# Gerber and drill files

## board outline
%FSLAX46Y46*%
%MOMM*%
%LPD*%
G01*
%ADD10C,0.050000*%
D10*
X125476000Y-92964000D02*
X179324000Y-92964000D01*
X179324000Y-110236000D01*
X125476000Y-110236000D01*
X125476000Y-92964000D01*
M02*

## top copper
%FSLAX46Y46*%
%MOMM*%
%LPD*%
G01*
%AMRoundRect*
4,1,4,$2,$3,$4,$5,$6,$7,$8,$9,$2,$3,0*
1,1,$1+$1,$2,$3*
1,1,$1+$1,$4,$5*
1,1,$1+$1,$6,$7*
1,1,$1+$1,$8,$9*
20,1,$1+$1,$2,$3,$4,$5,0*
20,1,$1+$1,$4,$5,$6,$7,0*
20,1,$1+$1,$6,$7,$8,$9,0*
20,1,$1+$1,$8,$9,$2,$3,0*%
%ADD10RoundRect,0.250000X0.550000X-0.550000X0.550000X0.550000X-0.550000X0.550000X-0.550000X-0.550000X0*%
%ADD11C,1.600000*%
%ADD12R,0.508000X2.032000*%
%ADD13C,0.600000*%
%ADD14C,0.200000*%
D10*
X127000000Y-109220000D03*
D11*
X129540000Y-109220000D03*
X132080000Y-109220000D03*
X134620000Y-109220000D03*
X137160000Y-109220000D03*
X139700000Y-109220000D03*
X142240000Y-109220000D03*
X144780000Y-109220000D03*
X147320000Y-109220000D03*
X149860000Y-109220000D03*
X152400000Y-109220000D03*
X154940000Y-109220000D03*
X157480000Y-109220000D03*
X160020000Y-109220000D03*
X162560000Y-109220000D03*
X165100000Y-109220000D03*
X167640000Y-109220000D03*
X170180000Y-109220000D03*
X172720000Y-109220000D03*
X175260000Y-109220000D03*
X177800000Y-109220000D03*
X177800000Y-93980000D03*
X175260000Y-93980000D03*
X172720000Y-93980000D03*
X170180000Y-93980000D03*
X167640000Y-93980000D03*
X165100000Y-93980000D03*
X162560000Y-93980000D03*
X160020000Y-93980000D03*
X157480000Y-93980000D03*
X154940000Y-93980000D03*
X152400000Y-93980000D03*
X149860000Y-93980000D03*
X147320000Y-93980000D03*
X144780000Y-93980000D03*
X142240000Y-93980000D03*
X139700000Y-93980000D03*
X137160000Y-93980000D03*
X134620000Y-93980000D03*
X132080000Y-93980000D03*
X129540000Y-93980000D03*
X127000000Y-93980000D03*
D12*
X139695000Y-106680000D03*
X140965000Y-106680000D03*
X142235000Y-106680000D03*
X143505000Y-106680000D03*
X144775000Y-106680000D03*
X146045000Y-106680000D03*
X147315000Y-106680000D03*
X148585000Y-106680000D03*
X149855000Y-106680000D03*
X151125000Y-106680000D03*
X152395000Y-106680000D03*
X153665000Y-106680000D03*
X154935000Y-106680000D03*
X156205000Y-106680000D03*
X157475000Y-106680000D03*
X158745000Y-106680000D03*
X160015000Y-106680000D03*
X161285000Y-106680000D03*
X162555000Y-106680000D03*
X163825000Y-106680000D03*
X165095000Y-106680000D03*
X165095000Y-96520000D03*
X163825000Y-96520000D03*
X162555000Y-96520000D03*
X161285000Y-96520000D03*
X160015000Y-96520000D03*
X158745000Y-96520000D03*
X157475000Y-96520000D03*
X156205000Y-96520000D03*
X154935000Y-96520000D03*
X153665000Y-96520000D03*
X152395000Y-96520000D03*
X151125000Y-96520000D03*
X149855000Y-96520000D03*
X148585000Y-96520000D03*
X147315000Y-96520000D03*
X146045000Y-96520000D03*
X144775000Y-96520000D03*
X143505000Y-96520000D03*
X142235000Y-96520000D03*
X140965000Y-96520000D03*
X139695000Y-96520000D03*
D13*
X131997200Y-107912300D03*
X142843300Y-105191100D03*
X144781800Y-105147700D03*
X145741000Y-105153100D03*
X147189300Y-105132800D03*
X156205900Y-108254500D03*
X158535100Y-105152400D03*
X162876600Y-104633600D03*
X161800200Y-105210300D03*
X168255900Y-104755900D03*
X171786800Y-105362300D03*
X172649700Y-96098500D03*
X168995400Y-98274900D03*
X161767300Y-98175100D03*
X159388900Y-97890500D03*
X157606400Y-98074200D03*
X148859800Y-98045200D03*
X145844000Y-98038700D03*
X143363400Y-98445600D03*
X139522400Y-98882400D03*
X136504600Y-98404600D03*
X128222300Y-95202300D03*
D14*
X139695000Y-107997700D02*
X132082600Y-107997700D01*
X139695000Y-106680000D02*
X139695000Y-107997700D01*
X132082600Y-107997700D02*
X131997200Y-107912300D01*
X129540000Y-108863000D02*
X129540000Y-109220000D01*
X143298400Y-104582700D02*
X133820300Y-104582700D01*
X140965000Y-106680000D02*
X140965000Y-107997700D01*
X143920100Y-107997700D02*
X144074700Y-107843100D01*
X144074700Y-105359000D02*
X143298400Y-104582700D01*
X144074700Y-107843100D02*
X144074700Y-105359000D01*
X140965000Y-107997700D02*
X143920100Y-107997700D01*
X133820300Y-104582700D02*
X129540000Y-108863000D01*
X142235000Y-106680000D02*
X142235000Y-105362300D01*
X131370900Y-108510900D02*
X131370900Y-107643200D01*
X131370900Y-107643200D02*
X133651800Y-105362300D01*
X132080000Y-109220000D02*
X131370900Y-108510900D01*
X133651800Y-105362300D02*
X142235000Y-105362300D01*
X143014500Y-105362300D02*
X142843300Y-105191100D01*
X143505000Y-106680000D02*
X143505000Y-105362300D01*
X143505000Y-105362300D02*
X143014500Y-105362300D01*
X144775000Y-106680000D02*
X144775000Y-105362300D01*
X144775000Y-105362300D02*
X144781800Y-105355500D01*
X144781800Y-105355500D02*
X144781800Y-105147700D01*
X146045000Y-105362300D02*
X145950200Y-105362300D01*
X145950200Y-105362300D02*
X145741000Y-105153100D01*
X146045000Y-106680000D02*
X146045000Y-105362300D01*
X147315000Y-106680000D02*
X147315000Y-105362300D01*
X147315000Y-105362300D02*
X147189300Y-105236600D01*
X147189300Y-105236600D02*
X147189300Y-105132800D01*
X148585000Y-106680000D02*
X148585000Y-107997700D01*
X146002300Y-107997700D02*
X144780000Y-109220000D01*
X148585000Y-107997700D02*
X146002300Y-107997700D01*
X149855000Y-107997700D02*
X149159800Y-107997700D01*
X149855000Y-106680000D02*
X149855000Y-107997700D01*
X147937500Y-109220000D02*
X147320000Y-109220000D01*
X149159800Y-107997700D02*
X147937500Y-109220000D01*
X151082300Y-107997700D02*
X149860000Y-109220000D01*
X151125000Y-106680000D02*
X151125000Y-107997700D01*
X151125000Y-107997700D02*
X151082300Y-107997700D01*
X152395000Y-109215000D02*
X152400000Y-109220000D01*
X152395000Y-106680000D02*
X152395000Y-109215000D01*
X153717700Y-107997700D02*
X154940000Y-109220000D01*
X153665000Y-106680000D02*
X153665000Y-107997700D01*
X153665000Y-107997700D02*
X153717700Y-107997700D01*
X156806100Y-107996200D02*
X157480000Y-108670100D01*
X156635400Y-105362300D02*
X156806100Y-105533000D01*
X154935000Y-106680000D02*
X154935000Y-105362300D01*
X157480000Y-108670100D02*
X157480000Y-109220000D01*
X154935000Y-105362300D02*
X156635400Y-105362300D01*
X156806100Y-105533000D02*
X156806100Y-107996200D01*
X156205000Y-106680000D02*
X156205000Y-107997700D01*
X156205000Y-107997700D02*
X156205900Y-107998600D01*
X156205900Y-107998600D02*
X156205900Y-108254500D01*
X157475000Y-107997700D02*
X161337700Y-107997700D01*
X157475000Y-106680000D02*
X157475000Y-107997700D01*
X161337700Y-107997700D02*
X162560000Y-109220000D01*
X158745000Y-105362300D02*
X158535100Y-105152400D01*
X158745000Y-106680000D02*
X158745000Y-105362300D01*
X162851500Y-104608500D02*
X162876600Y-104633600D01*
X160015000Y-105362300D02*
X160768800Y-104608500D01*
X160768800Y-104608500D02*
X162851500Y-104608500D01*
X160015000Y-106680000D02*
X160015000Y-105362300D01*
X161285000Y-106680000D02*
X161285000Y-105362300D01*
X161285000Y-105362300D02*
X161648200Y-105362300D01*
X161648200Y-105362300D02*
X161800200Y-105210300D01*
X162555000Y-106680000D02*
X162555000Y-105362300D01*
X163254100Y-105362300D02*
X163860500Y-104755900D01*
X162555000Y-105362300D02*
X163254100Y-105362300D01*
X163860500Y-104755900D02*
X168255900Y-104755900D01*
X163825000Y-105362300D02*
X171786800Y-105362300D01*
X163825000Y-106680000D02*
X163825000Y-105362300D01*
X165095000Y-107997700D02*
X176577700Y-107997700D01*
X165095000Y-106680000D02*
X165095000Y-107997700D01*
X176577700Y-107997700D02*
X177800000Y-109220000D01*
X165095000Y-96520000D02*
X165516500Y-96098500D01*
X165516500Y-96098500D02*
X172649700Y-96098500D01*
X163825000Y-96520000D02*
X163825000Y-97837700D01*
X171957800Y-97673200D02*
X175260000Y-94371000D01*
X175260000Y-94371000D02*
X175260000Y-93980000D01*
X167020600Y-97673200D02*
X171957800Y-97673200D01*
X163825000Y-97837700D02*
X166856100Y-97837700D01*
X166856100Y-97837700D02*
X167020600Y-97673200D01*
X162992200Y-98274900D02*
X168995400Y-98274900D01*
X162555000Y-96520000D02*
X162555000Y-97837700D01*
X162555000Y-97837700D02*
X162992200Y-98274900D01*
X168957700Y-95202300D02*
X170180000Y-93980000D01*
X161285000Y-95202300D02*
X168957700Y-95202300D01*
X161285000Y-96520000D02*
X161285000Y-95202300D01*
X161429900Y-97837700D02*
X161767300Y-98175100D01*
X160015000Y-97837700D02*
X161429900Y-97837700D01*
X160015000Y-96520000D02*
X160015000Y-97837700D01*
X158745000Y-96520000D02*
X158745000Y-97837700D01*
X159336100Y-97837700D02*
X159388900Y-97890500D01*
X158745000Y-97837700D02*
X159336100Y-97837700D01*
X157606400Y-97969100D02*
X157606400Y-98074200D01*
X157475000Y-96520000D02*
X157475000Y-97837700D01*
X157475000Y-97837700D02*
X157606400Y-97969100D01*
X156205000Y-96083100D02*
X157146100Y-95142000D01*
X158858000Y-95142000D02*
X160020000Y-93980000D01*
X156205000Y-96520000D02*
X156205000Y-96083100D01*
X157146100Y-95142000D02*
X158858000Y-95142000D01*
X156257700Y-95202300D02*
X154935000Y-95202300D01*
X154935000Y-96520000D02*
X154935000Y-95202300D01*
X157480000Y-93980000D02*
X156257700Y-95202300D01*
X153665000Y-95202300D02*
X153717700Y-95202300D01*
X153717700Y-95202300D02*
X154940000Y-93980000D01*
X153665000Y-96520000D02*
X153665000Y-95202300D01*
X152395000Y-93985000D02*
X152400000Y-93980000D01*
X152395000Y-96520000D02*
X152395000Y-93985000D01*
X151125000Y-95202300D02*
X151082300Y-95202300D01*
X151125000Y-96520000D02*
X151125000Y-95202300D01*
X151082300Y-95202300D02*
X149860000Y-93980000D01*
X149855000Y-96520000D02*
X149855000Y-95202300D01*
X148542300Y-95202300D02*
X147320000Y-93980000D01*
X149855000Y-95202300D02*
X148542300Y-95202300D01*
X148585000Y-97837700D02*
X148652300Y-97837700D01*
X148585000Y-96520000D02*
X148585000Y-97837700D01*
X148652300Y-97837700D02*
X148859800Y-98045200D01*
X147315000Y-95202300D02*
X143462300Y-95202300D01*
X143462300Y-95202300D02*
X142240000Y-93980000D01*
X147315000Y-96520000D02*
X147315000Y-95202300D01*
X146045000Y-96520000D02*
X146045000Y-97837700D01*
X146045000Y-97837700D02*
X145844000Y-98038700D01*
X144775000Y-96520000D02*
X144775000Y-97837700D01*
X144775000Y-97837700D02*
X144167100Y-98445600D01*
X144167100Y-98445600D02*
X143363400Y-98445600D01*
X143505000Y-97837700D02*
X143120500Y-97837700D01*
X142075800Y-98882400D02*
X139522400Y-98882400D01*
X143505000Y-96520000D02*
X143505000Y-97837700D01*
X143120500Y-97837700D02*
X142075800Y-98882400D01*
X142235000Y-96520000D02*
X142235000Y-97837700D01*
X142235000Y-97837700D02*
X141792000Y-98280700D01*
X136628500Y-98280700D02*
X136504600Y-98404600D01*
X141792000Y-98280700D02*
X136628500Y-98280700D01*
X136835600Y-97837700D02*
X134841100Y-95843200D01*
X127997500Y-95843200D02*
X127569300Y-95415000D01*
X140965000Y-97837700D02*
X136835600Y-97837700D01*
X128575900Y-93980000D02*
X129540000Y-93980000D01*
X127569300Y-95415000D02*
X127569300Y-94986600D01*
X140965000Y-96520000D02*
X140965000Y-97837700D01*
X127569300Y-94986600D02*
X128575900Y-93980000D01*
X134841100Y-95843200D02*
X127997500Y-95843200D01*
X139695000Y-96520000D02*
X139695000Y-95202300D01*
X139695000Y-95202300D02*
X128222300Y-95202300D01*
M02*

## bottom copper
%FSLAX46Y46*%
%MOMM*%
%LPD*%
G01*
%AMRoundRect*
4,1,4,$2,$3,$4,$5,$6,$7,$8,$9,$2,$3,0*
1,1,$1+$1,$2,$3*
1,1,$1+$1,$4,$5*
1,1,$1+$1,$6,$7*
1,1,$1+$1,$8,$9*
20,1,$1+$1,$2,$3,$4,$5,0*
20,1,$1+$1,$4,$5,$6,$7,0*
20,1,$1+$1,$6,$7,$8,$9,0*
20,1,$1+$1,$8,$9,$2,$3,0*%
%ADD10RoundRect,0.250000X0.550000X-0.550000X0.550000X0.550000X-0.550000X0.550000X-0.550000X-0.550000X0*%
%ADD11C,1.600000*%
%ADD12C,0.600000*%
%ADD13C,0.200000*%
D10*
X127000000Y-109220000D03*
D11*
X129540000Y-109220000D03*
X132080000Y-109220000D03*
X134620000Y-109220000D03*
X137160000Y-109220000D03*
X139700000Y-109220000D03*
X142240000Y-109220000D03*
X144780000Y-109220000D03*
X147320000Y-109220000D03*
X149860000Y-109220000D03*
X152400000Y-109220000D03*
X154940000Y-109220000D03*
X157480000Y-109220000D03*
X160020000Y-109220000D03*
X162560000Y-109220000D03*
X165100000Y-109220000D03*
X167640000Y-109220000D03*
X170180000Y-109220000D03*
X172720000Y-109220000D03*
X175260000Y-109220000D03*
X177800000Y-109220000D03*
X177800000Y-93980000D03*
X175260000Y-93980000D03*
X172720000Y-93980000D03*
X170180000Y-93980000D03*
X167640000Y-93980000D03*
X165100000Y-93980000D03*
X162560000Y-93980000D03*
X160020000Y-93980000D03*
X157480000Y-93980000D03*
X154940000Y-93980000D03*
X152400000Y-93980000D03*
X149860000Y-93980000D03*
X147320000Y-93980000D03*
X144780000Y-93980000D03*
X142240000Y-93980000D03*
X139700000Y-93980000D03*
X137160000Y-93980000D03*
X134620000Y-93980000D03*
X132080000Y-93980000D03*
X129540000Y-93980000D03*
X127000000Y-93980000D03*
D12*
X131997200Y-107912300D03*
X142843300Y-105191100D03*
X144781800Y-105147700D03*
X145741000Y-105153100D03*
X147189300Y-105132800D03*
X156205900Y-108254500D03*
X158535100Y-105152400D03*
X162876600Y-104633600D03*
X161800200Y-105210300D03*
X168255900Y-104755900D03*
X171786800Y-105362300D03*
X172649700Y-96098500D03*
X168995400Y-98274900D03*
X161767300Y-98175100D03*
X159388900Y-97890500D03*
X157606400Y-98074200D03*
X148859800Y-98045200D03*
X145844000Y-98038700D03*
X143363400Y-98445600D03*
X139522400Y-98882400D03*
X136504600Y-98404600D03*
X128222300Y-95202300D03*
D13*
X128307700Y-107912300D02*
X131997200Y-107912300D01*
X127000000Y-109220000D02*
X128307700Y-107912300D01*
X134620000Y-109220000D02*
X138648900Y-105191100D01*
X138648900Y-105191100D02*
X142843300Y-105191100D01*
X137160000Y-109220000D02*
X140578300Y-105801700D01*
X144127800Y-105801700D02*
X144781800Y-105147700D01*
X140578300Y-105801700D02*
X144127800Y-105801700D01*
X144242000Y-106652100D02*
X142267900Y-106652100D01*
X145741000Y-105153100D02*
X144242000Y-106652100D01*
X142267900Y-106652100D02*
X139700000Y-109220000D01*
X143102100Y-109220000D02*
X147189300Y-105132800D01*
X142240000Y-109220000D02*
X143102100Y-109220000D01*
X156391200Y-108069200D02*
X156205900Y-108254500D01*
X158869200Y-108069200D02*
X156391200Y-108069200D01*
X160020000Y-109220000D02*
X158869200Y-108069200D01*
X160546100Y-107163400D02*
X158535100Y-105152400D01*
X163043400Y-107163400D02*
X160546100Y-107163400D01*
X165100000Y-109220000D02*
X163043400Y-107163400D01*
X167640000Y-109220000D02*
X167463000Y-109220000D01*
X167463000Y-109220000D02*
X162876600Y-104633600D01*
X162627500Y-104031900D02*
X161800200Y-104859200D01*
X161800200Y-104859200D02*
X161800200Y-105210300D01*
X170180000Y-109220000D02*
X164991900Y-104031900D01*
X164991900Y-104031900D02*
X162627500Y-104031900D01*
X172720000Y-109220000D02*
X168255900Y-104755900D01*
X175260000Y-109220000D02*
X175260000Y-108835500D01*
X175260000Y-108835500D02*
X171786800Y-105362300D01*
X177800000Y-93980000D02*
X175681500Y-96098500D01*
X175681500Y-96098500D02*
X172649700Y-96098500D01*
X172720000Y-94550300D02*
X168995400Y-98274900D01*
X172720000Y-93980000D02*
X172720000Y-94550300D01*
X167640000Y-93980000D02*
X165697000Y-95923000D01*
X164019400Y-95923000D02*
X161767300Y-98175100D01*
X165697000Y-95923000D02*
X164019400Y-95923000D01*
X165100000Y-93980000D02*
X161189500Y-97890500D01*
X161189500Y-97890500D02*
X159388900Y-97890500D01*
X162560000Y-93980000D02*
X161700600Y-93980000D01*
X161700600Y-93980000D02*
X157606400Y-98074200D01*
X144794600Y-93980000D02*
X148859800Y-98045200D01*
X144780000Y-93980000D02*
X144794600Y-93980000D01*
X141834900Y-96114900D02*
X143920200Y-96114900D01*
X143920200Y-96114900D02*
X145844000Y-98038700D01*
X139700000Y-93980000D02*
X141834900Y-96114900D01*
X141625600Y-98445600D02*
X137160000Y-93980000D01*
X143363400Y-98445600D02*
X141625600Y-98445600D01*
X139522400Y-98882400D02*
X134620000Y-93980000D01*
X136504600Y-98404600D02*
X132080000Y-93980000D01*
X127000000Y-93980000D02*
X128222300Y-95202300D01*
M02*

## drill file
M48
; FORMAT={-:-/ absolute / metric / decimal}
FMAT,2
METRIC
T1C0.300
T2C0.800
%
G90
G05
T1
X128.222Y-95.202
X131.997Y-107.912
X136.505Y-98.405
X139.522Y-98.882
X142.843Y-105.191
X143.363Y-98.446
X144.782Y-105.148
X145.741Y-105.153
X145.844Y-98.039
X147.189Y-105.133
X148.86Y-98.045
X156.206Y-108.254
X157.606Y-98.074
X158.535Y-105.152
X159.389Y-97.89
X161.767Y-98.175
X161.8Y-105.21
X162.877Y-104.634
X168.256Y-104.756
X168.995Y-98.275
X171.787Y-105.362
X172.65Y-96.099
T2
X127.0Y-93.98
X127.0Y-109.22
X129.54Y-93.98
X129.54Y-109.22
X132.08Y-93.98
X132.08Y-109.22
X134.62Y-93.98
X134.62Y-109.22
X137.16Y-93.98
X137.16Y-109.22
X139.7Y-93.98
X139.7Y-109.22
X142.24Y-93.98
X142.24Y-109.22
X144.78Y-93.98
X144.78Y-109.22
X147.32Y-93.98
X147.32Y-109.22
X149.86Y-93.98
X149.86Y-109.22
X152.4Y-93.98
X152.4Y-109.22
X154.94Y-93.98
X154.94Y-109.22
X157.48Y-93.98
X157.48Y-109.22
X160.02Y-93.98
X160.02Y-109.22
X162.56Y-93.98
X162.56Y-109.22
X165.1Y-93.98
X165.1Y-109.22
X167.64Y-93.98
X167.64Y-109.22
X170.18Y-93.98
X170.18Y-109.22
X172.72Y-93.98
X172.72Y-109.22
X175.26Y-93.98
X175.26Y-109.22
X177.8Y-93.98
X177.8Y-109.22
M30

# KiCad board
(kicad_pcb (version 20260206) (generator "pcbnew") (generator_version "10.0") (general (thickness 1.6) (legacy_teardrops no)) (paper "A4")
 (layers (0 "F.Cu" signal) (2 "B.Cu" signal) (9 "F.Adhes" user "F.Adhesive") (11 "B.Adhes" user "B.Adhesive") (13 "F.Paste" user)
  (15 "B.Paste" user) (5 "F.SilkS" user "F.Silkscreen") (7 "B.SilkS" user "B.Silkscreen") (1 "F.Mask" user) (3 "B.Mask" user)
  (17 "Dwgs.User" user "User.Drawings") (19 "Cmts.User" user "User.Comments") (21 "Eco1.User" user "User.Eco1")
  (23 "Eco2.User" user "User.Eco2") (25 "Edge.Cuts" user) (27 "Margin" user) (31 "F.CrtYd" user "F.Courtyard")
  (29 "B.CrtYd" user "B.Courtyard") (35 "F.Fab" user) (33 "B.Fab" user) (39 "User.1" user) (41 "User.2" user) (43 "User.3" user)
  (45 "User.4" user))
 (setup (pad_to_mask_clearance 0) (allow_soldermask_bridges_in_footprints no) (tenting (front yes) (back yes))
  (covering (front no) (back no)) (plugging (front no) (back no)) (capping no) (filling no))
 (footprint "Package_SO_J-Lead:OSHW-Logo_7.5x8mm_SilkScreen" (layer "F.Cu") (at 152.5 101.5)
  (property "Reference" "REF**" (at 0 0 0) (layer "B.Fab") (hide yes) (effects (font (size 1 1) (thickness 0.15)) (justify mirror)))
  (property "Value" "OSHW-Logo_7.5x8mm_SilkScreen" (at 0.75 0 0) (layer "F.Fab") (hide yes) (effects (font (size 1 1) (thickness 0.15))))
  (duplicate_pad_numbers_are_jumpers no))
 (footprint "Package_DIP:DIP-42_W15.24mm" (layer "F.Cu") (at 127 109.22 90)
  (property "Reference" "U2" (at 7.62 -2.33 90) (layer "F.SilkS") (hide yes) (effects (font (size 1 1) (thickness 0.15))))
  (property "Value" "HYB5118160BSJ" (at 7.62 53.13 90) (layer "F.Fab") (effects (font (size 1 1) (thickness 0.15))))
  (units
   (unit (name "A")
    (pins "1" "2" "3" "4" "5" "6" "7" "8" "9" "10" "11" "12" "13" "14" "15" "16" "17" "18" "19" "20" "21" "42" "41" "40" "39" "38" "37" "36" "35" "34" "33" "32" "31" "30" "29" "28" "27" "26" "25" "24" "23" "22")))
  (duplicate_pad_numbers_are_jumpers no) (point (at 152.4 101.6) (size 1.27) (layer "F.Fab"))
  (pad "1" thru_hole roundrect (at 0 0 90) (size 1.6 1.6) (drill 0.8) (layers "*.Cu" "*.Mask") (remove_unused_layers no)
   (roundrect_rratio 0.15625) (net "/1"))
  (pad "2" thru_hole circle (at 0 2.54 90) (size 1.6 1.6) (drill 0.8) (layers "*.Cu" "*.Mask") (remove_unused_layers no) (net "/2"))
  (pad "3" thru_hole circle (at 0 5.08 90) (size 1.6 1.6) (drill 0.8) (layers "*.Cu" "*.Mask") (remove_unused_layers no) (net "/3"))
  (pad "4" thru_hole circle (at 0 7.62 90) (size 1.6 1.6) (drill 0.8) (layers "*.Cu" "*.Mask") (remove_unused_layers no) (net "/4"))
  (pad "5" thru_hole circle (at 0 10.16 90) (size 1.6 1.6) (drill 0.8) (layers "*.Cu" "*.Mask") (remove_unused_layers no) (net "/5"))
  (pad "6" thru_hole circle (at 0 12.7 90) (size 1.6 1.6) (drill 0.8) (layers "*.Cu" "*.Mask") (remove_unused_layers no) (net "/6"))
  (pad "7" thru_hole circle (at 0 15.24 90) (size 1.6 1.6) (drill 0.8) (layers "*.Cu" "*.Mask") (remove_unused_layers no) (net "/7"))
  (pad "8" thru_hole circle (at 0 17.78 90) (size 1.6 1.6) (drill 0.8) (layers "*.Cu" "*.Mask") (remove_unused_layers no) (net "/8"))
  (pad "9" thru_hole circle (at 0 20.32 90) (size 1.6 1.6) (drill 0.8) (layers "*.Cu" "*.Mask") (remove_unused_layers no) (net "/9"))
  (pad "10" thru_hole circle (at 0 22.86 90) (size 1.6 1.6) (drill 0.8) (layers "*.Cu" "*.Mask") (remove_unused_layers no) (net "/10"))
  (pad "11" thru_hole circle (at 0 25.4 90) (size 1.6 1.6) (drill 0.8) (layers "*.Cu" "*.Mask") (remove_unused_layers no) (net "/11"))
  (pad "12" thru_hole circle (at 0 27.94 90) (size 1.6 1.6) (drill 0.8) (layers "*.Cu" "*.Mask") (remove_unused_layers no) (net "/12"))
  (pad "13" thru_hole circle (at 0 30.48 90) (size 1.6 1.6) (drill 0.8) (layers "*.Cu" "*.Mask") (remove_unused_layers no) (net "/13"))
  (pad "14" thru_hole circle (at 0 33.02 90) (size 1.6 1.6) (drill 0.8) (layers "*.Cu" "*.Mask") (remove_unused_layers no) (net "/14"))
  (pad "15" thru_hole circle (at 0 35.56 90) (size 1.6 1.6) (drill 0.8) (layers "*.Cu" "*.Mask") (remove_unused_layers no) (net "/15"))
  (pad "16" thru_hole circle (at 0 38.1 90) (size 1.6 1.6) (drill 0.8) (layers "*.Cu" "*.Mask") (remove_unused_layers no) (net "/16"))
  (pad "17" thru_hole circle (at 0 40.64 90) (size 1.6 1.6) (drill 0.8) (layers "*.Cu" "*.Mask") (remove_unused_layers no) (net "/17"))
  (pad "18" thru_hole circle (at 0 43.18 90) (size 1.6 1.6) (drill 0.8) (layers "*.Cu" "*.Mask") (remove_unused_layers no) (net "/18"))
  (pad "19" thru_hole circle (at 0 45.72 90) (size 1.6 1.6) (drill 0.8) (layers "*.Cu" "*.Mask") (remove_unused_layers no) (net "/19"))
  (pad "20" thru_hole circle (at 0 48.26 90) (size 1.6 1.6) (drill 0.8) (layers "*.Cu" "*.Mask") (remove_unused_layers no) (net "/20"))
  (pad "21" thru_hole circle (at 0 50.8 90) (size 1.6 1.6) (drill 0.8) (layers "*.Cu" "*.Mask") (remove_unused_layers no) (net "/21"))
  (pad "22" thru_hole circle (at 15.24 50.8 90) (size 1.6 1.6) (drill 0.8) (layers "*.Cu" "*.Mask") (remove_unused_layers no) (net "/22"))
  (pad "23" thru_hole circle (at 15.24 48.26 90) (size 1.6 1.6) (drill 0.8) (layers "*.Cu" "*.Mask") (remove_unused_layers no) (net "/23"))
  (pad "24" thru_hole circle (at 15.24 45.72 90) (size 1.6 1.6) (drill 0.8) (layers "*.Cu" "*.Mask") (remove_unused_layers no) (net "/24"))
  (pad "25" thru_hole circle (at 15.24 43.18 90) (size 1.6 1.6) (drill 0.8) (layers "*.Cu" "*.Mask") (remove_unused_layers no) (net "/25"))
  (pad "26" thru_hole circle (at 15.24 40.64 90) (size 1.6 1.6) (drill 0.8) (layers "*.Cu" "*.Mask") (remove_unused_layers no) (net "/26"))
  (pad "27" thru_hole circle (at 15.24 38.1 90) (size 1.6 1.6) (drill 0.8) (layers "*.Cu" "*.Mask") (remove_unused_layers no) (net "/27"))
  (pad "28" thru_hole circle (at 15.24 35.56 90) (size 1.6 1.6) (drill 0.8) (layers "*.Cu" "*.Mask") (remove_unused_layers no) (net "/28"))
  (pad "29" thru_hole circle (at 15.24 33.02 90) (size 1.6 1.6) (drill 0.8) (layers "*.Cu" "*.Mask") (remove_unused_layers no) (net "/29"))
  (pad "30" thru_hole circle (at 15.24 30.48 90) (size 1.6 1.6) (drill 0.8) (layers "*.Cu" "*.Mask") (remove_unused_layers no) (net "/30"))
  (pad "31" thru_hole circle (at 15.24 27.94 90) (size 1.6 1.6) (drill 0.8) (layers "*.Cu" "*.Mask") (remove_unused_layers no) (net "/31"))
  (pad "32" thru_hole circle (at 15.24 25.4 90) (size 1.6 1.6) (drill 0.8) (layers "*.Cu" "*.Mask") (remove_unused_layers no) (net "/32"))
  (pad "33" thru_hole circle (at 15.24 22.86 90) (size 1.6 1.6) (drill 0.8) (layers "*.Cu" "*.Mask") (remove_unused_layers no) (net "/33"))
  (pad "34" thru_hole circle (at 15.24 20.32 90) (size 1.6 1.6) (drill 0.8) (layers "*.Cu" "*.Mask") (remove_unused_layers no) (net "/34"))
  (pad "35" thru_hole circle (at 15.24 17.78 90) (size 1.6 1.6) (drill 0.8) (layers "*.Cu" "*.Mask") (remove_unused_layers no) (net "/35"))
  (pad "36" thru_hole circle (at 15.24 15.24 90) (size 1.6 1.6) (drill 0.8) (layers "*.Cu" "*.Mask") (remove_unused_layers no) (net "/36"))
  (pad "37" thru_hole circle (at 15.24 12.7 90) (size 1.6 1.6) (drill 0.8) (layers "*.Cu" "*.Mask") (remove_unused_layers no) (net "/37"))
  (pad "38" thru_hole circle (at 15.24 10.16 90) (size 1.6 1.6) (drill 0.8) (layers "*.Cu" "*.Mask") (remove_unused_layers no) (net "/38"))
  (pad "39" thru_hole circle (at 15.24 7.62 90) (size 1.6 1.6) (drill 0.8) (layers "*.Cu" "*.Mask") (remove_unused_layers no) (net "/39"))
  (pad "40" thru_hole circle (at 15.24 5.08 90) (size 1.6 1.6) (drill 0.8) (layers "*.Cu" "*.Mask") (remove_unused_layers no) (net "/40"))
  (pad "41" thru_hole circle (at 15.24 2.54 90) (size 1.6 1.6) (drill 0.8) (layers "*.Cu" "*.Mask") (remove_unused_layers no) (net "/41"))
  (pad "42" thru_hole circle (at 15.24 0 90) (size 1.6 1.6) (drill 0.8) (layers "*.Cu" "*.Mask") (remove_unused_layers no) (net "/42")))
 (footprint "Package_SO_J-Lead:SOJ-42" (layer "F.Cu") (at 152.395 101.6)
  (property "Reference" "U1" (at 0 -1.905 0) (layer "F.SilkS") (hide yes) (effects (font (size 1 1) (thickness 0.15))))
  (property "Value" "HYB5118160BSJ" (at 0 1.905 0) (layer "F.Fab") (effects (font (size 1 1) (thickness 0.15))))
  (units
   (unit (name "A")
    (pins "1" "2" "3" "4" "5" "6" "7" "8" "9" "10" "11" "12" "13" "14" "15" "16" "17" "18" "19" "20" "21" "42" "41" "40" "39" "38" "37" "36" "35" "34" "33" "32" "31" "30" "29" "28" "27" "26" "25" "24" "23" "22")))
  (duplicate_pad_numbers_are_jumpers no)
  (pad "1" smd rect (at -12.7 5.08) (size 0.508 2.032) (layers "F.Cu" "F.Mask" "F.Paste") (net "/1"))
  (pad "2" smd rect (at -11.43 5.08) (size 0.508 2.032) (layers "F.Cu" "F.Mask" "F.Paste") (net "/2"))
  (pad "3" smd rect (at -10.16 5.08) (size 0.508 2.032) (layers "F.Cu" "F.Mask" "F.Paste") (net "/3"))
  (pad "4" smd rect (at -8.89 5.08) (size 0.508 2.032) (layers "F.Cu" "F.Mask" "F.Paste") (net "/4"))
  (pad "5" smd rect (at -7.62 5.08) (size 0.508 2.032) (layers "F.Cu" "F.Mask" "F.Paste") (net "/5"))
  (pad "6" smd rect (at -6.35 5.08) (size 0.508 2.032) (layers "F.Cu" "F.Mask" "F.Paste") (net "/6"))
  (pad "7" smd rect (at -5.08 5.08) (size 0.508 2.032) (layers "F.Cu" "F.Mask" "F.Paste") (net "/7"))
  (pad "8" smd rect (at -3.81 5.08) (size 0.508 2.032) (layers "F.Cu" "F.Mask" "F.Paste") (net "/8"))
  (pad "9" smd rect (at -2.54 5.08) (size 0.508 2.032) (layers "F.Cu" "F.Mask" "F.Paste") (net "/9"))
  (pad "10" smd rect (at -1.27 5.08) (size 0.508 2.032) (layers "F.Cu" "F.Mask" "F.Paste") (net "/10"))
  (pad "11" smd rect (at 0 5.08) (size 0.508 2.032) (layers "F.Cu" "F.Mask" "F.Paste") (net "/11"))
  (pad "12" smd rect (at 1.27 5.08) (size 0.508 2.032) (layers "F.Cu" "F.Mask" "F.Paste") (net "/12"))
  (pad "13" smd rect (at 2.54 5.08) (size 0.508 2.032) (layers "F.Cu" "F.Mask" "F.Paste") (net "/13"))
  (pad "14" smd rect (at 3.81 5.08) (size 0.508 2.032) (layers "F.Cu" "F.Mask" "F.Paste") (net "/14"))
  (pad "15" smd rect (at 5.08 5.08) (size 0.508 2.032) (layers "F.Cu" "F.Mask" "F.Paste") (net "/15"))
  (pad "16" smd rect (at 6.35 5.08) (size 0.508 2.032) (layers "F.Cu" "F.Mask" "F.Paste") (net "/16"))
  (pad "17" smd rect (at 7.62 5.08) (size 0.508 2.032) (layers "F.Cu" "F.Mask" "F.Paste") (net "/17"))
  (pad "18" smd rect (at 8.89 5.08) (size 0.508 2.032) (layers "F.Cu" "F.Mask" "F.Paste") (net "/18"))
  (pad "19" smd rect (at 10.16 5.08) (size 0.508 2.032) (layers "F.Cu" "F.Mask" "F.Paste") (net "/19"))
  (pad "20" smd rect (at 11.43 5.08) (size 0.508 2.032) (layers "F.Cu" "F.Mask" "F.Paste") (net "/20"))
  (pad "21" smd rect (at 12.7 5.08) (size 0.508 2.032) (layers "F.Cu" "F.Mask" "F.Paste") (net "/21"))
  (pad "22" smd rect (at 12.7 -5.08) (size 0.508 2.032) (layers "F.Cu" "F.Mask" "F.Paste") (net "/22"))
  (pad "23" smd rect (at 11.43 -5.08) (size 0.508 2.032) (layers "F.Cu" "F.Mask" "F.Paste") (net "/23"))
  (pad "24" smd rect (at 10.16 -5.08) (size 0.508 2.032) (layers "F.Cu" "F.Mask" "F.Paste") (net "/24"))
  (pad "25" smd rect (at 8.89 -5.08) (size 0.508 2.032) (layers "F.Cu" "F.Mask" "F.Paste") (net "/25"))
  (pad "26" smd rect (at 7.62 -5.08) (size 0.508 2.032) (layers "F.Cu" "F.Mask" "F.Paste") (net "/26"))
  (pad "27" smd rect (at 6.35 -5.08) (size 0.508 2.032) (layers "F.Cu" "F.Mask" "F.Paste") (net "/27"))
  (pad "28" smd rect (at 5.08 -5.08) (size 0.508 2.032) (layers "F.Cu" "F.Mask" "F.Paste") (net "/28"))
  (pad "29" smd rect (at 3.81 -5.08) (size 0.508 2.032) (layers "F.Cu" "F.Mask" "F.Paste") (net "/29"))
  (pad "30" smd rect (at 2.54 -5.08) (size 0.508 2.032) (layers "F.Cu" "F.Mask" "F.Paste") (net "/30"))
  (pad "31" smd rect (at 1.27 -5.08) (size 0.508 2.032) (layers "F.Cu" "F.Mask" "F.Paste") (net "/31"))
  (pad "32" smd rect (at 0 -5.08) (size 0.508 2.032) (layers "F.Cu" "F.Mask" "F.Paste") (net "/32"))
  (pad "33" smd rect (at -1.27 -5.08) (size 0.508 2.032) (layers "F.Cu" "F.Mask" "F.Paste") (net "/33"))
  (pad "34" smd rect (at -2.54 -5.08) (size 0.508 2.032) (layers "F.Cu" "F.Mask" "F.Paste") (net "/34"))
  (pad "35" smd rect (at -3.81 -5.08) (size 0.508 2.032) (layers "F.Cu" "F.Mask" "F.Paste") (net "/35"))
  (pad "36" smd rect (at -5.08 -5.08) (size 0.508 2.032) (layers "F.Cu" "F.Mask" "F.Paste") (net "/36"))
  (pad "37" smd rect (at -6.35 -5.08) (size 0.508 2.032) (layers "F.Cu" "F.Mask" "F.Paste") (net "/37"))
  (pad "38" smd rect (at -7.62 -5.08) (size 0.508 2.032) (layers "F.Cu" "F.Mask" "F.Paste") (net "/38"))
  (pad "39" smd rect (at -8.89 -5.08) (size 0.508 2.032) (layers "F.Cu" "F.Mask" "F.Paste") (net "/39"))
  (pad "40" smd rect (at -10.16 -5.08) (size 0.508 2.032) (layers "F.Cu" "F.Mask" "F.Paste") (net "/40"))
  (pad "41" smd rect (at -11.43 -5.08) (size 0.508 2.032) (layers "F.Cu" "F.Mask" "F.Paste") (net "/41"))
  (pad "42" smd rect (at -12.7 -5.08) (size 0.508 2.032) (layers "F.Cu" "F.Mask" "F.Paste") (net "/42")))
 (gr_rect (start 125.476 92.964) (end 179.324 110.236) (stroke (width 0.05) (type default)) (fill no) (layer "Edge.Cuts"))
 (segment (start 139.695 107.9977) (end 132.0826 107.9977) (width 0.2) (layer "F.Cu") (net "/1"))
 (segment (start 139.695 106.68) (end 139.695 107.9977) (width 0.2) (layer "F.Cu") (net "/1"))
 (segment (start 132.0826 107.9977) (end 131.9972 107.9123) (width 0.2) (layer "F.Cu") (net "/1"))
 (via (at 131.9972 107.9123) (size 0.6) (drill 0.3) (layers "F.Cu" "B.Cu") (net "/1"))
 (segment (start 128.3077 107.9123) (end 131.9972 107.9123) (width 0.2) (layer "B.Cu") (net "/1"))
 (segment (start 127 109.22) (end 128.3077 107.9123) (width 0.2) (layer "B.Cu") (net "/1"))
 (segment (start 129.54 108.863) (end 129.54 109.22) (width 0.2) (layer "F.Cu") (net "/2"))
 (segment (start 143.2984 104.5827) (end 133.8203 104.5827) (width 0.2) (layer "F.Cu") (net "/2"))
 (segment (start 140.965 106.68) (end 140.965 107.9977) (width 0.2) (layer "F.Cu") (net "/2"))
 (segment (start 143.9201 107.9977) (end 144.0747 107.8431) (width 0.2) (layer "F.Cu") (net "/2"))
 (segment (start 144.0747 105.359) (end 143.2984 104.5827) (width 0.2) (layer "F.Cu") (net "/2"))
 (segment (start 144.0747 107.8431) (end 144.0747 105.359) (width 0.2) (layer "F.Cu") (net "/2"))
 (segment (start 140.965 107.9977) (end 143.9201 107.9977) (width 0.2) (layer "F.Cu") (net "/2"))
 (segment (start 133.8203 104.5827) (end 129.54 108.863) (width 0.2) (layer "F.Cu") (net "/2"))
 (segment (start 142.235 106.68) (end 142.235 105.3623) (width 0.2) (layer "F.Cu") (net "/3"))
 (segment (start 131.3709 108.5109) (end 131.3709 107.6432) (width 0.2) (layer "F.Cu") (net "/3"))
 (segment (start 131.3709 107.6432) (end 133.6518 105.3623) (width 0.2) (layer "F.Cu") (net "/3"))
 (segment (start 132.08 109.22) (end 131.3709 108.5109) (width 0.2) (layer "F.Cu") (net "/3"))
 (segment (start 133.6518 105.3623) (end 142.235 105.3623) (width 0.2) (layer "F.Cu") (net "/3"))
 (segment (start 143.0145 105.3623) (end 142.8433 105.1911) (width 0.2) (layer "F.Cu") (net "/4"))
 (segment (start 143.505 106.68) (end 143.505 105.3623) (width 0.2) (layer "F.Cu") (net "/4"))
 (segment (start 143.505 105.3623) (end 143.0145 105.3623) (width 0.2) (layer "F.Cu") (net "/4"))
 (via (at 142.8433 105.1911) (size 0.6) (drill 0.3) (layers "F.Cu" "B.Cu") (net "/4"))
 (segment (start 134.62 109.22) (end 138.6489 105.1911) (width 0.2) (layer "B.Cu") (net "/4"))
 (segment (start 138.6489 105.1911) (end 142.8433 105.1911) (width 0.2) (layer "B.Cu") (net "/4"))
 (segment (start 144.775 106.68) (end 144.775 105.3623) (width 0.2) (layer "F.Cu") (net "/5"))
 (segment (start 144.775 105.3623) (end 144.7818 105.3555) (width 0.2) (layer "F.Cu") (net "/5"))
 (segment (start 144.7818 105.3555) (end 144.7818 105.1477) (width 0.2) (layer "F.Cu") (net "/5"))
 (via (at 144.7818 105.1477) (size 0.6) (drill 0.3) (layers "F.Cu" "B.Cu") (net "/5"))
 (segment (start 137.16 109.22) (end 140.5783 105.8017) (width 0.2) (layer "B.Cu") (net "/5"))
 (segment (start 144.1278 105.8017) (end 144.7818 105.1477) (width 0.2) (layer "B.Cu") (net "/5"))
 (segment (start 140.5783 105.8017) (end 144.1278 105.8017) (width 0.2) (layer "B.Cu") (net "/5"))
 (segment (start 146.045 105.3623) (end 145.9502 105.3623) (width 0.2) (layer "F.Cu") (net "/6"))
 (segment (start 145.9502 105.3623) (end 145.741 105.1531) (width 0.2) (layer "F.Cu") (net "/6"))
 (segment (start 146.045 106.68) (end 146.045 105.3623) (width 0.2) (layer "F.Cu") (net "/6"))
 (via (at 145.741 105.1531) (size 0.6) (drill 0.3) (layers "F.Cu" "B.Cu") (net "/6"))
 (segment (start 144.242 106.6521) (end 142.2679 106.6521) (width 0.2) (layer "B.Cu") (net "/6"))
 (segment (start 145.741 105.1531) (end 144.242 106.6521) (width 0.2) (layer "B.Cu") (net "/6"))
 (segment (start 142.2679 106.6521) (end 139.7 109.22) (width 0.2) (layer "B.Cu") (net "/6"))
 (segment (start 147.315 106.68) (end 147.315 105.3623) (width 0.2) (layer "F.Cu") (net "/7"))
 (segment (start 147.315 105.3623) (end 147.1893 105.2366) (width 0.2) (layer "F.Cu") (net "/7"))
 (segment (start 147.1893 105.2366) (end 147.1893 105.1328) (width 0.2) (layer "F.Cu") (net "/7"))
 (via (at 147.1893 105.1328) (size 0.6) (drill 0.3) (layers "F.Cu" "B.Cu") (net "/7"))
 (segment (start 143.1021 109.22) (end 147.1893 105.1328) (width 0.2) (layer "B.Cu") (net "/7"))
 (segment (start 142.24 109.22) (end 143.1021 109.22) (width 0.2) (layer "B.Cu") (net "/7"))
 (segment (start 148.585 106.68) (end 148.585 107.9977) (width 0.2) (layer "F.Cu") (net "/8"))
 (segment (start 146.0023 107.9977) (end 144.78 109.22) (width 0.2) (layer "F.Cu") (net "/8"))
 (segment (start 148.585 107.9977) (end 146.0023 107.9977) (width 0.2) (layer "F.Cu") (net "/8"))
 (segment (start 149.855 107.9977) (end 149.1598 107.9977) (width 0.2) (layer "F.Cu") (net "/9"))
 (segment (start 149.855 106.68) (end 149.855 107.9977) (width 0.2) (layer "F.Cu") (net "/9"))
 (segment (start 147.9375 109.22) (end 147.32 109.22) (width 0.2) (layer "F.Cu") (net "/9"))
 (segment (start 149.1598 107.9977) (end 147.9375 109.22) (width 0.2) (layer "F.Cu") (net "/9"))
 (segment (start 151.0823 107.9977) (end 149.86 109.22) (width 0.2) (layer "F.Cu") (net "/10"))
 (segment (start 151.125 106.68) (end 151.125 107.9977) (width 0.2) (layer "F.Cu") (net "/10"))
 (segment (start 151.125 107.9977) (end 151.0823 107.9977) (width 0.2) (layer "F.Cu") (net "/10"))
 (segment (start 152.395 109.215) (end 152.4 109.22) (width 0.2) (layer "F.Cu") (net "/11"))
 (segment (start 152.395 106.68) (end 152.395 109.215) (width 0.2) (layer "F.Cu") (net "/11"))
 (segment (start 153.7177 107.9977) (end 154.94 109.22) (width 0.2) (layer "F.Cu") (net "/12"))
 (segment (start 153.665 106.68) (end 153.665 107.9977) (width 0.2) (layer "F.Cu") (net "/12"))
 (segment (start 153.665 107.9977) (end 153.7177 107.9977) (width 0.2) (layer "F.Cu") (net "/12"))
 (segment (start 156.8061 107.9962) (end 157.48 108.6701) (width 0.2) (layer "F.Cu") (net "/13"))
 (segment (start 156.6354 105.3623) (end 156.8061 105.533) (width 0.2) (layer "F.Cu") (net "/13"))
 (segment (start 154.935 106.68) (end 154.935 105.3623) (width 0.2) (layer "F.Cu") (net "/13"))
 (segment (start 157.48 108.6701) (end 157.48 109.22) (width 0.2) (layer "F.Cu") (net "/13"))
 (segment (start 154.935 105.3623) (end 156.6354 105.3623) (width 0.2) (layer "F.Cu") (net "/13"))
 (segment (start 156.8061 105.533) (end 156.8061 107.9962) (width 0.2) (layer "F.Cu") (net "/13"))
 (segment (start 156.205 106.68) (end 156.205 107.9977) (width 0.2) (layer "F.Cu") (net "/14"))
 (segment (start 156.205 107.9977) (end 156.2059 107.9986) (width 0.2) (layer "F.Cu") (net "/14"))
 (segment (start 156.2059 107.9986) (end 156.2059 108.2545) (width 0.2) (layer "F.Cu") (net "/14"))
 (via (at 156.2059 108.2545) (size 0.6) (drill 0.3) (layers "F.Cu" "B.Cu") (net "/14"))
 (segment (start 156.3912 108.0692) (end 156.2059 108.2545) (width 0.2) (layer "B.Cu") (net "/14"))
 (segment (start 158.8692 108.0692) (end 156.3912 108.0692) (width 0.2) (layer "B.Cu") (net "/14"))
 (segment (start 160.02 109.22) (end 158.8692 108.0692) (width 0.2) (layer "B.Cu") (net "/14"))
 (segment (start 157.475 107.9977) (end 161.3377 107.9977) (width 0.2) (layer "F.Cu") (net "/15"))
 (segment (start 157.475 106.68) (end 157.475 107.9977) (width 0.2) (layer "F.Cu") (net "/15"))
 (segment (start 161.3377 107.9977) (end 162.56 109.22) (width 0.2) (layer "F.Cu") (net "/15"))
 (segment (start 158.745 105.3623) (end 158.5351 105.1524) (width 0.2) (layer "F.Cu") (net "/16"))
 (segment (start 158.745 106.68) (end 158.745 105.3623) (width 0.2) (layer "F.Cu") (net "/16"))
 (via (at 158.5351 105.1524) (size 0.6) (drill 0.3) (layers "F.Cu" "B.Cu") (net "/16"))
 (segment (start 160.5461 107.1634) (end 158.5351 105.1524) (width 0.2) (layer "B.Cu") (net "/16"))
 (segment (start 163.0434 107.1634) (end 160.5461 107.1634) (width 0.2) (layer "B.Cu") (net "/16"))
 (segment (start 165.1 109.22) (end 163.0434 107.1634) (width 0.2) (layer "B.Cu") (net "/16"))
 (segment (start 162.8515 104.6085) (end 162.8766 104.6336) (width 0.2) (layer "F.Cu") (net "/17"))
 (segment (start 160.015 105.3623) (end 160.7688 104.6085) (width 0.2) (layer "F.Cu") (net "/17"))
 (segment (start 160.7688 104.6085) (end 162.8515 104.6085) (width 0.2) (layer "F.Cu") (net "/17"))
 (segment (start 160.015 106.68) (end 160.015 105.3623) (width 0.2) (layer "F.Cu") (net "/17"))
 (via (at 162.8766 104.6336) (size 0.6) (drill 0.3) (layers "F.Cu" "B.Cu") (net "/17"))
 (segment (start 167.64 109.22) (end 167.463 109.22) (width 0.2) (layer "B.Cu") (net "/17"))
 (segment (start 167.463 109.22) (end 162.8766 104.6336) (width 0.2) (layer "B.Cu") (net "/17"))
 (segment (start 161.285 106.68) (end 161.285 105.3623) (width 0.2) (layer "F.Cu") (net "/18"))
 (segment (start 161.285 105.3623) (end 161.6482 105.3623) (width 0.2) (layer "F.Cu") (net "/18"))
 (segment (start 161.6482 105.3623) (end 161.8002 105.2103) (width 0.2) (layer "F.Cu") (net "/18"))
 (via (at 161.8002 105.2103) (size 0.6) (drill 0.3) (layers "F.Cu" "B.Cu") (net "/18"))
 (segment (start 162.6275 104.0319) (end 161.8002 104.8592) (width 0.2) (layer "B.Cu") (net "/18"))
 (segment (start 161.8002 104.8592) (end 161.8002 105.2103) (width 0.2) (layer "B.Cu") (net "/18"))
 (segment (start 170.18 109.22) (end 164.9919 104.0319) (width 0.2) (layer "B.Cu") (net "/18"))
 (segment (start 164.9919 104.0319) (end 162.6275 104.0319) (width 0.2) (layer "B.Cu") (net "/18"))
 (segment (start 162.555 106.68) (end 162.555 105.3623) (width 0.2) (layer "F.Cu") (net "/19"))
 (segment (start 163.2541 105.3623) (end 163.8605 104.7559) (width 0.2) (layer "F.Cu") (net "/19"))
 (segment (start 162.555 105.3623) (end 163.2541 105.3623) (width 0.2) (layer "F.Cu") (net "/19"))
 (segment (start 163.8605 104.7559) (end 168.2559 104.7559) (width 0.2) (layer "F.Cu") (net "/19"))
 (via (at 168.2559 104.7559) (size 0.6) (drill 0.3) (layers "F.Cu" "B.Cu") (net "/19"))
 (segment (start 172.72 109.22) (end 168.2559 104.7559) (width 0.2) (layer "B.Cu") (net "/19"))
 (segment (start 163.825 105.3623) (end 171.7868 105.3623) (width 0.2) (layer "F.Cu") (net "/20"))
 (segment (start 163.825 106.68) (end 163.825 105.3623) (width 0.2) (layer "F.Cu") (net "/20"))
 (via (at 171.7868 105.3623) (size 0.6) (drill 0.3) (layers "F.Cu" "B.Cu") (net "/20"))
 (segment (start 175.26 109.22) (end 175.26 108.8355) (width 0.2) (layer "B.Cu") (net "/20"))
 (segment (start 175.26 108.8355) (end 171.7868 105.3623) (width 0.2) (layer "B.Cu") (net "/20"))
 (segment (start 165.095 107.9977) (end 176.5777 107.9977) (width 0.2) (layer "F.Cu") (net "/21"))
 (segment (start 165.095 106.68) (end 165.095 107.9977) (width 0.2) (layer "F.Cu") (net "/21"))
 (segment (start 176.5777 107.9977) (end 177.8 109.22) (width 0.2) (layer "F.Cu") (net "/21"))
 (segment (start 165.095 96.52) (end 165.5165 96.0985) (width 0.2) (layer "F.Cu") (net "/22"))
 (segment (start 165.5165 96.0985) (end 172.6497 96.0985) (width 0.2) (layer "F.Cu") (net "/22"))
 (via (at 172.6497 96.0985) (size 0.6) (drill 0.3) (layers "F.Cu" "B.Cu") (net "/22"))
 (segment (start 177.8 93.98) (end 175.6815 96.0985) (width 0.2) (layer "B.Cu") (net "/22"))
 (segment (start 175.6815 96.0985) (end 172.6497 96.0985) (width 0.2) (layer "B.Cu") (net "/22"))
 (segment (start 163.825 96.52) (end 163.825 97.8377) (width 0.2) (layer "F.Cu") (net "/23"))
 (segment (start 171.9578 97.6732) (end 175.26 94.371) (width 0.2) (layer "F.Cu") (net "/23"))
 (segment (start 175.26 94.371) (end 175.26 93.98) (width 0.2) (layer "F.Cu") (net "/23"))
 (segment (start 167.0206 97.6732) (end 171.9578 97.6732) (width 0.2) (layer "F.Cu") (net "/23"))
 (segment (start 163.825 97.8377) (end 166.8561 97.8377) (width 0.2) (layer "F.Cu") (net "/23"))
 (segment (start 166.8561 97.8377) (end 167.0206 97.6732) (width 0.2) (layer "F.Cu") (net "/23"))
 (segment (start 162.9922 98.2749) (end 168.9954 98.2749) (width 0.2) (layer "F.Cu") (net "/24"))
 (segment (start 162.555 96.52) (end 162.555 97.8377) (width 0.2) (layer "F.Cu") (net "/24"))
 (segment (start 162.555 97.8377) (end 162.9922 98.2749) (width 0.2) (layer "F.Cu") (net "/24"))
 (via (at 168.9954 98.2749) (size 0.6) (drill 0.3) (layers "F.Cu" "B.Cu") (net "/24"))
 (segment (start 172.72 94.5503) (end 168.9954 98.2749) (width 0.2) (layer "B.Cu") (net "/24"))
 (segment (start 172.72 93.98) (end 172.72 94.5503) (width 0.2) (layer "B.Cu") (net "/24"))
 (segment (start 168.9577 95.2023) (end 170.18 93.98) (width 0.2) (layer "F.Cu") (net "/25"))
 (segment (start 161.285 95.2023) (end 168.9577 95.2023) (width 0.2) (layer "F.Cu") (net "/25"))
 (segment (start 161.285 96.52) (end 161.285 95.2023) (width 0.2) (layer "F.Cu") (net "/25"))
 (segment (start 161.4299 97.8377) (end 161.7673 98.1751) (width 0.2) (layer "F.Cu") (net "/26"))
 (segment (start 160.015 97.8377) (end 161.4299 97.8377) (width 0.2) (layer "F.Cu") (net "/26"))
 (segment (start 160.015 96.52) (end 160.015 97.8377) (width 0.2) (layer "F.Cu") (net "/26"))
 (via (at 161.7673 98.1751) (size 0.6) (drill 0.3) (layers "F.Cu" "B.Cu") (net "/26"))
 (segment (start 167.64 93.98) (end 165.697 95.923) (width 0.2) (layer "B.Cu") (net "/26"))
 (segment (start 164.0194 95.923) (end 161.7673 98.1751) (width 0.2) (layer "B.Cu") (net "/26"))
 (segment (start 165.697 95.923) (end 164.0194 95.923) (width 0.2) (layer "B.Cu") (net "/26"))
 (segment (start 158.745 96.52) (end 158.745 97.8377) (width 0.2) (layer "F.Cu") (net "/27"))
 (segment (start 159.3361 97.8377) (end 159.3889 97.8905) (width 0.2) (layer "F.Cu") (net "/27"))
 (segment (start 158.745 97.8377) (end 159.3361 97.8377) (width 0.2) (layer "F.Cu") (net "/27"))
 (via (at 159.3889 97.8905) (size 0.6) (drill 0.3) (layers "F.Cu" "B.Cu") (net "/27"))
 (segment (start 165.1 93.98) (end 161.1895 97.8905) (width 0.2) (layer "B.Cu") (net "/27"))
 (segment (start 161.1895 97.8905) (end 159.3889 97.8905) (width 0.2) (layer "B.Cu") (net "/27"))
 (segment (start 157.6064 97.9691) (end 157.6064 98.0742) (width 0.2) (layer "F.Cu") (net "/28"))
 (segment (start 157.475 96.52) (end 157.475 97.8377) (width 0.2) (layer "F.Cu") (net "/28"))
 (segment (start 157.475 97.8377) (end 157.6064 97.9691) (width 0.2) (layer "F.Cu") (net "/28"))
 (via (at 157.6064 98.0742) (size 0.6) (drill 0.3) (layers "F.Cu" "B.Cu") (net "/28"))
 (segment (start 162.56 93.98) (end 161.7006 93.98) (width 0.2) (layer "B.Cu") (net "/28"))
 (segment (start 161.7006 93.98) (end 157.6064 98.0742) (width 0.2) (layer "B.Cu") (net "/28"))
 (segment (start 156.205 96.0831) (end 157.1461 95.142) (width 0.2) (layer "F.Cu") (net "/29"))
 (segment (start 158.858 95.142) (end 160.02 93.98) (width 0.2) (layer "F.Cu") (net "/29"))
 (segment (start 156.205 96.52) (end 156.205 96.0831) (width 0.2) (layer "F.Cu") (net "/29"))
 (segment (start 157.1461 95.142) (end 158.858 95.142) (width 0.2) (layer "F.Cu") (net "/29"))
 (segment (start 156.2577 95.2023) (end 154.935 95.2023) (width 0.2) (layer "F.Cu") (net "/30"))
 (segment (start 154.935 96.52) (end 154.935 95.2023) (width 0.2) (layer "F.Cu") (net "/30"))
 (segment (start 157.48 93.98) (end 156.2577 95.2023) (width 0.2) (layer "F.Cu") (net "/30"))
 (segment (start 153.665 95.2023) (end 153.7177 95.2023) (width 0.2) (layer "F.Cu") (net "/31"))
 (segment (start 153.7177 95.2023) (end 154.94 93.98) (width 0.2) (layer "F.Cu") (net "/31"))
 (segment (start 153.665 96.52) (end 153.665 95.2023) (width 0.2) (layer "F.Cu") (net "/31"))
 (segment (start 152.395 93.985) (end 152.4 93.98) (width 0.2) (layer "F.Cu") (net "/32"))
 (segment (start 152.395 96.52) (end 152.395 93.985) (width 0.2) (layer "F.Cu") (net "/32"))
 (segment (start 151.125 95.2023) (end 151.0823 95.2023) (width 0.2) (layer "F.Cu") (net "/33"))
 (segment (start 151.125 96.52) (end 151.125 95.2023) (width 0.2) (layer "F.Cu") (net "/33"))
 (segment (start 151.0823 95.2023) (end 149.86 93.98) (width 0.2) (layer "F.Cu") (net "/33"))
 (segment (start 149.855 96.52) (end 149.855 95.2023) (width 0.2) (layer "F.Cu") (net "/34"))
 (segment (start 148.5423 95.2023) (end 147.32 93.98) (width 0.2) (layer "F.Cu") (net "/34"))
 (segment (start 149.855 95.2023) (end 148.5423 95.2023) (width 0.2) (layer "F.Cu") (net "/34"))
 (segment (start 148.585 97.8377) (end 148.6523 97.8377) (width 0.2) (layer "F.Cu") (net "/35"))
 (segment (start 148.585 96.52) (end 148.585 97.8377) (width 0.2) (layer "F.Cu") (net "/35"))
 (segment (start 148.6523 97.8377) (end 148.8598 98.0452) (width 0.2) (layer "F.Cu") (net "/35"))
 (via (at 148.8598 98.0452) (size 0.6) (drill 0.3) (layers "F.Cu" "B.Cu") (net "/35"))
 (segment (start 144.7946 93.98) (end 148.8598 98.0452) (width 0.2) (layer "B.Cu") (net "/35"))
 (segment (start 144.78 93.98) (end 144.7946 93.98) (width 0.2) (layer "B.Cu") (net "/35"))
 (segment (start 147.315 95.2023) (end 143.4623 95.2023) (width 0.2) (layer "F.Cu") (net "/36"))
 (segment (start 143.4623 95.2023) (end 142.24 93.98) (width 0.2) (layer "F.Cu") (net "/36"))
 (segment (start 147.315 96.52) (end 147.315 95.2023) (width 0.2) (layer "F.Cu") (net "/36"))
 (segment (start 146.045 96.52) (end 146.045 97.8377) (width 0.2) (layer "F.Cu") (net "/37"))
 (segment (start 146.045 97.8377) (end 145.844 98.0387) (width 0.2) (layer "F.Cu") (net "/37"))
 (via (at 145.844 98.0387) (size 0.6) (drill 0.3) (layers "F.Cu" "B.Cu") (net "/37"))
 (segment (start 141.8349 96.1149) (end 143.9202 96.1149) (width 0.2) (layer "B.Cu") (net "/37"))
 (segment (start 143.9202 96.1149) (end 145.844 98.0387) (width 0.2) (layer "B.Cu") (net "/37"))
 (segment (start 139.7 93.98) (end 141.8349 96.1149) (width 0.2) (layer "B.Cu") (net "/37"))
 (segment (start 144.775 96.52) (end 144.775 97.8377) (width 0.2) (layer "F.Cu") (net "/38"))
 (segment (start 144.775 97.8377) (end 144.1671 98.4456) (width 0.2) (layer "F.Cu") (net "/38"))
 (segment (start 144.1671 98.4456) (end 143.3634 98.4456) (width 0.2) (layer "F.Cu") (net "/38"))
 (via (at 143.3634 98.4456) (size 0.6) (drill 0.3) (layers "F.Cu" "B.Cu") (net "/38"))
 (segment (start 141.6256 98.4456) (end 137.16 93.98) (width 0.2) (layer "B.Cu") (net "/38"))
 (segment (start 143.3634 98.4456) (end 141.6256 98.4456) (width 0.2) (layer "B.Cu") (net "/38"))
 (segment (start 143.505 97.8377) (end 143.1205 97.8377) (width 0.2) (layer "F.Cu") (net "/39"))
 (segment (start 142.0758 98.8824) (end 139.5224 98.8824) (width 0.2) (layer "F.Cu") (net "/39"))
 (segment (start 143.505 96.52) (end 143.505 97.8377) (width 0.2) (layer "F.Cu") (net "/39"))
 (segment (start 143.1205 97.8377) (end 142.0758 98.8824) (width 0.2) (layer "F.Cu") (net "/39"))
 (via (at 139.5224 98.8824) (size 0.6) (drill 0.3) (layers "F.Cu" "B.Cu") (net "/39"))
 (segment (start 139.5224 98.8824) (end 134.62 93.98) (width 0.2) (layer "B.Cu") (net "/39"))
 (segment (start 142.235 96.52) (end 142.235 97.8377) (width 0.2) (layer "F.Cu") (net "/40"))
 (segment (start 142.235 97.8377) (end 141.792 98.2807) (width 0.2) (layer "F.Cu") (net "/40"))
 (segment (start 136.6285 98.2807) (end 136.5046 98.4046) (width 0.2) (layer "F.Cu") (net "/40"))
 (segment (start 141.792 98.2807) (end 136.6285 98.2807) (width 0.2) (layer "F.Cu") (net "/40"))
 (via (at 136.5046 98.4046) (size 0.6) (drill 0.3) (layers "F.Cu" "B.Cu") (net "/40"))
 (segment (start 136.5046 98.4046) (end 132.08 93.98) (width 0.2) (layer "B.Cu") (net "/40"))
 (segment (start 136.8356 97.8377) (end 134.8411 95.8432) (width 0.2) (layer "F.Cu") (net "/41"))
 (segment (start 127.9975 95.8432) (end 127.5693 95.415) (width 0.2) (layer "F.Cu") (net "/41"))
 (segment (start 140.965 97.8377) (end 136.8356 97.8377) (width 0.2) (layer "F.Cu") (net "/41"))
 (segment (start 128.5759 93.98) (end 129.54 93.98) (width 0.2) (layer "F.Cu") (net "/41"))
 (segment (start 127.5693 95.415) (end 127.5693 94.9866) (width 0.2) (layer "F.Cu") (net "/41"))
 (segment (start 140.965 96.52) (end 140.965 97.8377) (width 0.2) (layer "F.Cu") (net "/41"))
 (segment (start 127.5693 94.9866) (end 128.5759 93.98) (width 0.2) (layer "F.Cu") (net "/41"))
 (segment (start 134.8411 95.8432) (end 127.9975 95.8432) (width 0.2) (layer "F.Cu") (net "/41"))
 (segment (start 139.695 96.52) (end 139.695 95.2023) (width 0.2) (layer "F.Cu") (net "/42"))
 (segment (start 139.695 95.2023) (end 128.2223 95.2023) (width 0.2) (layer "F.Cu") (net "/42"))
 (via (at 128.2223 95.2023) (size 0.6) (drill 0.3) (layers "F.Cu" "B.Cu") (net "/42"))
 (segment (start 127 93.98) (end 128.2223 95.2023) (width 0.2) (layer "B.Cu") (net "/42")))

